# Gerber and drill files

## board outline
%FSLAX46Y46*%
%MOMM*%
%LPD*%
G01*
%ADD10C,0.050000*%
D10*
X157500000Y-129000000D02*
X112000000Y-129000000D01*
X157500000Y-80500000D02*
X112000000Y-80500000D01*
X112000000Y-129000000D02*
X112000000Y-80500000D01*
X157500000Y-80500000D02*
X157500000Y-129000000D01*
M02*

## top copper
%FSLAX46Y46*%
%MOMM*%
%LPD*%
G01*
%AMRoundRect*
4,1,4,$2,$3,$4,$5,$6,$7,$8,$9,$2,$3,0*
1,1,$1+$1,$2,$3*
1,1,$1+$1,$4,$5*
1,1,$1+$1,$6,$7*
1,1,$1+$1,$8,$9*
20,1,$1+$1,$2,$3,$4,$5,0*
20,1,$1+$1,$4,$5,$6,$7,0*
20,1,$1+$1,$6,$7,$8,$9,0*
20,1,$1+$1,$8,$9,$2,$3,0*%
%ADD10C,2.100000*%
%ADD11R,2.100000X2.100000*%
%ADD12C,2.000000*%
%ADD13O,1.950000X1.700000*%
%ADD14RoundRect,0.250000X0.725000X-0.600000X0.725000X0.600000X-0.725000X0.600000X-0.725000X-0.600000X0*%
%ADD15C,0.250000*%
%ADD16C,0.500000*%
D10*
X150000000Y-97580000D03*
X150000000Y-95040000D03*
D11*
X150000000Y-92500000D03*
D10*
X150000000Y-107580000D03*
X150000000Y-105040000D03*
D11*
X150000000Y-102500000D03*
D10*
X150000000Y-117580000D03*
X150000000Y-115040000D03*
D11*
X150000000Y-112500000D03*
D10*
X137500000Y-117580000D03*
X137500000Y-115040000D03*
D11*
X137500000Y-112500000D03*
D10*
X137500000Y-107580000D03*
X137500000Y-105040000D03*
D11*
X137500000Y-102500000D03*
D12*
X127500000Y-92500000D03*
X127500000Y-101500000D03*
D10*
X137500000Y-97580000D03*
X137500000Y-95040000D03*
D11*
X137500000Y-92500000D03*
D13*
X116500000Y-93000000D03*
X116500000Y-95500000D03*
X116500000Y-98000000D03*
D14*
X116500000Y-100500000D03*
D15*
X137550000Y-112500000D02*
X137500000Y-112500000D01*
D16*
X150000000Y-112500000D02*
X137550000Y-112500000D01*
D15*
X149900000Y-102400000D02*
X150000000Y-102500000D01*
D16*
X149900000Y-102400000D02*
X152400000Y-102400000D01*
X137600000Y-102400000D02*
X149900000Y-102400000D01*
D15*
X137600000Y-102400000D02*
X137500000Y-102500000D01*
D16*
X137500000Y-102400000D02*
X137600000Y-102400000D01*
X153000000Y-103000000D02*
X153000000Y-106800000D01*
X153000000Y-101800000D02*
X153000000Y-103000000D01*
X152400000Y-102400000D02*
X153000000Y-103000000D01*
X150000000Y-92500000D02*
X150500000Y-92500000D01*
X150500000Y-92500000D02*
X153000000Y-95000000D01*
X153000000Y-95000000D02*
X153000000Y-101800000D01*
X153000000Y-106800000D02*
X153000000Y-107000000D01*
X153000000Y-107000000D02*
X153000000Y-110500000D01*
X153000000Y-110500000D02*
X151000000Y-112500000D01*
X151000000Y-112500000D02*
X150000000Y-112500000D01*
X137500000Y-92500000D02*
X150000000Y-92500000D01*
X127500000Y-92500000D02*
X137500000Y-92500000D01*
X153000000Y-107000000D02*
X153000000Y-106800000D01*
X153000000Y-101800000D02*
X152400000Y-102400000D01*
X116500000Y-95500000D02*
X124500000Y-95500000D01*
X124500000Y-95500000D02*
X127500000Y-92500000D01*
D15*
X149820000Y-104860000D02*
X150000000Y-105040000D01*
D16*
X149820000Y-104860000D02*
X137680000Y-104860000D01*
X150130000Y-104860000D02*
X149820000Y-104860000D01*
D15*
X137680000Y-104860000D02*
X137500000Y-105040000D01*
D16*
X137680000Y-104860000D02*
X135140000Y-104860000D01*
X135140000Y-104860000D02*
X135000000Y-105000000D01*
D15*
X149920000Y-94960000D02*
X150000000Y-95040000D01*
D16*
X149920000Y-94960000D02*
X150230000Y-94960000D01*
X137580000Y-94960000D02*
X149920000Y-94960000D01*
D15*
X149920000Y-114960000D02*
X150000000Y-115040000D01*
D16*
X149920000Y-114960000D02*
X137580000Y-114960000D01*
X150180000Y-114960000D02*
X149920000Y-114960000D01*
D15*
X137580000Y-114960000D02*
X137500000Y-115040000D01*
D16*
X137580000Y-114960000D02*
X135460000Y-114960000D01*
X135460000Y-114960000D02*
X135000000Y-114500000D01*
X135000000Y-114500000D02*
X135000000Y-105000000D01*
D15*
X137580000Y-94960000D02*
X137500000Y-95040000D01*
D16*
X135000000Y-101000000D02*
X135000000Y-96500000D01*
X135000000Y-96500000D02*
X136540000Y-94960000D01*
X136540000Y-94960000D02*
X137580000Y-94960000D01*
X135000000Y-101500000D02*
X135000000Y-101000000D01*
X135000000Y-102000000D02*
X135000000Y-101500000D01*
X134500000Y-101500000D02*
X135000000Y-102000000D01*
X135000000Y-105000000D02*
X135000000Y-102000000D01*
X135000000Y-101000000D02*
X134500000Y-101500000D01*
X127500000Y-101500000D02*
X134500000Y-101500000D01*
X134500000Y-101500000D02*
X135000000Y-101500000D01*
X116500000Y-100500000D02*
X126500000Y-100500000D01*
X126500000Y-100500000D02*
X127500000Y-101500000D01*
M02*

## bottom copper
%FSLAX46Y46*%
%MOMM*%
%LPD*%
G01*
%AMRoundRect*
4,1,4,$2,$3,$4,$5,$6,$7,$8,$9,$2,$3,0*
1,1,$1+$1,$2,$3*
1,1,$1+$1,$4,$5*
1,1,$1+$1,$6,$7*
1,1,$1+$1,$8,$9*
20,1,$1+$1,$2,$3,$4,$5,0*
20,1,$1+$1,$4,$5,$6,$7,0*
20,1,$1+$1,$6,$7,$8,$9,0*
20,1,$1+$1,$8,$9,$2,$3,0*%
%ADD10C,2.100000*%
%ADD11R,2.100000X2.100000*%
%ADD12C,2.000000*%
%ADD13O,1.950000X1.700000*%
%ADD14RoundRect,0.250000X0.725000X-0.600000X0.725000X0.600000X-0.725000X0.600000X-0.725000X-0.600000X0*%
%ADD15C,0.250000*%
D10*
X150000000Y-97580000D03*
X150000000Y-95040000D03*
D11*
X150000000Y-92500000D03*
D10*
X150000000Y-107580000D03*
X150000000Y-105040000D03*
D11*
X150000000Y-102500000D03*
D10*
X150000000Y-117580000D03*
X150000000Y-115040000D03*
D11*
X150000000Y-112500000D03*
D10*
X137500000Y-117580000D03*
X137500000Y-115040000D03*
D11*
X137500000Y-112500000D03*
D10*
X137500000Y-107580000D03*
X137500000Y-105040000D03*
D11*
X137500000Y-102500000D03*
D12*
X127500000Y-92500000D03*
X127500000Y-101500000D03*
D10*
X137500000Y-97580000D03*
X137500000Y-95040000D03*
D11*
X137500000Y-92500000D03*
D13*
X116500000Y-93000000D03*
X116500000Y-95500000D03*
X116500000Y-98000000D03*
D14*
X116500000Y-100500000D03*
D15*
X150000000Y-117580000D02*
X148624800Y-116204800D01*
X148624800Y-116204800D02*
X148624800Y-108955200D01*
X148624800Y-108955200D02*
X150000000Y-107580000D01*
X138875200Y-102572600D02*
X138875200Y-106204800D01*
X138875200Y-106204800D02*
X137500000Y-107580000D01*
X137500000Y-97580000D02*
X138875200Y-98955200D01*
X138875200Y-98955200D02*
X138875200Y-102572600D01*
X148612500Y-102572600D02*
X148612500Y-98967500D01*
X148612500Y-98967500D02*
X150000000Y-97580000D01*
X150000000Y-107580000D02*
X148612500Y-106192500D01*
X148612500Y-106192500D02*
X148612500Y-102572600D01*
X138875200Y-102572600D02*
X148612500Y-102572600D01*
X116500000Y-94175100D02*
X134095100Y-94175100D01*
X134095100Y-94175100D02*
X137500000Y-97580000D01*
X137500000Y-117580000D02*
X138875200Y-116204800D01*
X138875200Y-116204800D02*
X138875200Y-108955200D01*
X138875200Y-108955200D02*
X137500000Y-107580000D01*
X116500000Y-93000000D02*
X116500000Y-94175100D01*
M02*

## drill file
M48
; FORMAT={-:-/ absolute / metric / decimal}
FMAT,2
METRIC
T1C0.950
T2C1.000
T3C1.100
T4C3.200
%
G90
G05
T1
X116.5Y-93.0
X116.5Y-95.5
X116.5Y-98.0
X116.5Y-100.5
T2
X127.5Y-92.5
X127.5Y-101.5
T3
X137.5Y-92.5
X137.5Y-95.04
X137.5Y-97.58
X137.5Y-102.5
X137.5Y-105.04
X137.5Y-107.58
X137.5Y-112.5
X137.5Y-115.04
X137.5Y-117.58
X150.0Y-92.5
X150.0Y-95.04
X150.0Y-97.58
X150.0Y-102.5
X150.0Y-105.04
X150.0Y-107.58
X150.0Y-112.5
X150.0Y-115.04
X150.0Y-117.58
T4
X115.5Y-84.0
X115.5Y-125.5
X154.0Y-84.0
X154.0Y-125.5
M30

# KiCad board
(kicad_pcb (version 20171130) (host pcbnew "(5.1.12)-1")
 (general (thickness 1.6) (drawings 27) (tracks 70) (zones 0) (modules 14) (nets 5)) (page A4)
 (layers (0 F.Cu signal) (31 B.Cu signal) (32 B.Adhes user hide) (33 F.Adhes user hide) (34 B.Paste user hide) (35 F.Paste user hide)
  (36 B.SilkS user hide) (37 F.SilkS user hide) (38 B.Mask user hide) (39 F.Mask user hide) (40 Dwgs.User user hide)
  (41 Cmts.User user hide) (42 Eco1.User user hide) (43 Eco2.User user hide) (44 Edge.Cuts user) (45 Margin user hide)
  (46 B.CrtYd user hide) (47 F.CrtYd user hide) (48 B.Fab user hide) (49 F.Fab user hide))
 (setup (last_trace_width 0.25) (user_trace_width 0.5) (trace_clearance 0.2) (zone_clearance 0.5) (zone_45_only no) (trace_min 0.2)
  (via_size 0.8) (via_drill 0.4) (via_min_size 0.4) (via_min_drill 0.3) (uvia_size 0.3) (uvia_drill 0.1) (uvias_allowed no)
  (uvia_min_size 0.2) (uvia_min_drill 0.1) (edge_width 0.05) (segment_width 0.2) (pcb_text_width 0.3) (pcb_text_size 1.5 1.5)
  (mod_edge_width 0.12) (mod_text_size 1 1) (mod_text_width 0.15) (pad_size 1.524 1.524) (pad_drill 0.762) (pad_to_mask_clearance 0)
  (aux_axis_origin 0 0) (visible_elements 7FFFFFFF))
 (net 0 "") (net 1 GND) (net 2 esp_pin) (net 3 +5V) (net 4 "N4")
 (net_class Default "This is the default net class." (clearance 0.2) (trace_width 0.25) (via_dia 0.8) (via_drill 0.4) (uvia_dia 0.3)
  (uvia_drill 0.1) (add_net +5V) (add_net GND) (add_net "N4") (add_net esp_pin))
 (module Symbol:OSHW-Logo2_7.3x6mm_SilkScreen (layer F.Cu) (at 137.5 124.5)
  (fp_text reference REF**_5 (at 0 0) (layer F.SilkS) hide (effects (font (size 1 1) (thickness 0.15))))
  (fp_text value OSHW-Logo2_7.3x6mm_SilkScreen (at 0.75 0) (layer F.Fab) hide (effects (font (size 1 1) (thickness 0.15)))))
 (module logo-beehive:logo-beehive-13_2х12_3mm (layer F.Cu) (at 123 109.22)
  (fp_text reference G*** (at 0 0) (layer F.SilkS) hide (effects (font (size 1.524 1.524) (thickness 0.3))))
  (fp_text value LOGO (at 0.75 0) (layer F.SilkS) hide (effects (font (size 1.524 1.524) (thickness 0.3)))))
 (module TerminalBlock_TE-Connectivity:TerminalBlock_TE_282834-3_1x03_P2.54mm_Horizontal (layer F.Cu) (at 150 92.5 270)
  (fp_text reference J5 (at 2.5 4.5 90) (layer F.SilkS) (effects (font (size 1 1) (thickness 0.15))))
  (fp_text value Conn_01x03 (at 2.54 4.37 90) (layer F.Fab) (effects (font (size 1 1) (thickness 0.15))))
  (pad 3 thru_hole circle (at 5.08 0 270) (size 2.1 2.1) (drill 1.1) (layers *.Cu *.Mask) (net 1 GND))
  (pad 2 thru_hole circle (at 2.54 0 270) (size 2.1 2.1) (drill 1.1) (layers *.Cu *.Mask) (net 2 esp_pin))
  (pad 1 thru_hole rect (at 0 0 270) (size 2.1 2.1) (drill 1.1) (layers *.Cu *.Mask) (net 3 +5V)))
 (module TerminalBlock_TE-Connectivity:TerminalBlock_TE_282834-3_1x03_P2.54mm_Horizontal (layer F.Cu) (at 150 102.5 270)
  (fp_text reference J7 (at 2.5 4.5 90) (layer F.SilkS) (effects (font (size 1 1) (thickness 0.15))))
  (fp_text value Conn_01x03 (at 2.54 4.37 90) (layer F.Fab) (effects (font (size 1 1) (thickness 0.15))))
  (pad 3 thru_hole circle (at 5.08 0 270) (size 2.1 2.1) (drill 1.1) (layers *.Cu *.Mask) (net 1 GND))
  (pad 2 thru_hole circle (at 2.54 0 270) (size 2.1 2.1) (drill 1.1) (layers *.Cu *.Mask) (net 2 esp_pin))
  (pad 1 thru_hole rect (at 0 0 270) (size 2.1 2.1) (drill 1.1) (layers *.Cu *.Mask) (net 3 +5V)))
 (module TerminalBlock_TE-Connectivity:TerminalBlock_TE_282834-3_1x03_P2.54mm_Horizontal (layer F.Cu) (at 150 112.5 270)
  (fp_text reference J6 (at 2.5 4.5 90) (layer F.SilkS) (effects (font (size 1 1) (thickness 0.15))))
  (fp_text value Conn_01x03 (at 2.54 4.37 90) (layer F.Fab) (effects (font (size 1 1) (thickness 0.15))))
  (pad 3 thru_hole circle (at 5.08 0 270) (size 2.1 2.1) (drill 1.1) (layers *.Cu *.Mask) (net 1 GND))
  (pad 2 thru_hole circle (at 2.54 0 270) (size 2.1 2.1) (drill 1.1) (layers *.Cu *.Mask) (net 2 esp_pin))
  (pad 1 thru_hole rect (at 0 0 270) (size 2.1 2.1) (drill 1.1) (layers *.Cu *.Mask) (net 3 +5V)))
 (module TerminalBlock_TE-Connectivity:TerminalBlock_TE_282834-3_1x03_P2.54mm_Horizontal (layer F.Cu) (at 137.5 112.5 270)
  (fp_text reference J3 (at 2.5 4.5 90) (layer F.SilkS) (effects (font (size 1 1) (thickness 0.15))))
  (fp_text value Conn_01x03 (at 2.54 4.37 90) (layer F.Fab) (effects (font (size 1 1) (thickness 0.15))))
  (pad 3 thru_hole circle (at 5.08 0 270) (size 2.1 2.1) (drill 1.1) (layers *.Cu *.Mask) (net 1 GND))
  (pad 2 thru_hole circle (at 2.54 0 270) (size 2.1 2.1) (drill 1.1) (layers *.Cu *.Mask) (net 2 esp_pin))
  (pad 1 thru_hole rect (at 0 0 270) (size 2.1 2.1) (drill 1.1) (layers *.Cu *.Mask) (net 3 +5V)))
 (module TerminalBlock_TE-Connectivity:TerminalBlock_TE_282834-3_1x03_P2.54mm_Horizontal (layer F.Cu) (at 137.5 102.5 270)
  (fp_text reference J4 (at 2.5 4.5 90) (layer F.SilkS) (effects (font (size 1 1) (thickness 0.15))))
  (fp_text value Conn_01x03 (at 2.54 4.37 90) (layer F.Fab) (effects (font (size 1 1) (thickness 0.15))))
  (pad 3 thru_hole circle (at 5.08 0 270) (size 2.1 2.1) (drill 1.1) (layers *.Cu *.Mask) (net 1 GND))
  (pad 2 thru_hole circle (at 2.54 0 270) (size 2.1 2.1) (drill 1.1) (layers *.Cu *.Mask) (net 2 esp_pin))
  (pad 1 thru_hole rect (at 0 0 270) (size 2.1 2.1) (drill 1.1) (layers *.Cu *.Mask) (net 3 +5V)))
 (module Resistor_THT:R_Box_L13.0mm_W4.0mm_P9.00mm (layer F.Cu) (at 127.5 101.5 90)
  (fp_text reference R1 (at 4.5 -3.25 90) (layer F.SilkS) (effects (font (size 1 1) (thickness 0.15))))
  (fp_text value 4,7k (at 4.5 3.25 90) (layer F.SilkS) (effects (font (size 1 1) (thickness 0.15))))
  (pad 2 thru_hole circle (at 9 0 90) (size 2 2) (drill 1) (layers *.Cu *.Mask) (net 3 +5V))
  (pad 1 thru_hole circle (at 0 0 90) (size 2 2) (drill 1) (layers *.Cu *.Mask) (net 2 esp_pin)))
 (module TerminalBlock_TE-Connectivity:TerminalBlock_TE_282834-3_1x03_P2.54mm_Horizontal (layer F.Cu) (at 137.5 92.5 270)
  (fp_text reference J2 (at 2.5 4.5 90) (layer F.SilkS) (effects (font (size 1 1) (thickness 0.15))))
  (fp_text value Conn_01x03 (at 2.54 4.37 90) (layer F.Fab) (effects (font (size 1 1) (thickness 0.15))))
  (pad 3 thru_hole circle (at 5.08 0 270) (size 2.1 2.1) (drill 1.1) (layers *.Cu *.Mask) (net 1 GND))
  (pad 2 thru_hole circle (at 2.54 0 270) (size 2.1 2.1) (drill 1.1) (layers *.Cu *.Mask) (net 2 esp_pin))
  (pad 1 thru_hole rect (at 0 0 270) (size 2.1 2.1) (drill 1.1) (layers *.Cu *.Mask) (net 3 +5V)))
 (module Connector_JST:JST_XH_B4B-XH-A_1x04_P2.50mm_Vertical (layer F.Cu) (at 116.5 100.5 90)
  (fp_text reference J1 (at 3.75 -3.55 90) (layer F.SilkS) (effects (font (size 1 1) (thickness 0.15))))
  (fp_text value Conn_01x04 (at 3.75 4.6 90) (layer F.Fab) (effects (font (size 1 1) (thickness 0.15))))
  (pad 4 thru_hole oval (at 7.5 0 90) (size 1.7 1.95) (drill 0.95) (layers *.Cu *.Mask) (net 1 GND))
  (pad 3 thru_hole oval (at 5 0 90) (size 1.7 1.95) (drill 0.95) (layers *.Cu *.Mask) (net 3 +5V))
  (pad 2 thru_hole oval (at 2.5 0 90) (size 1.7 1.95) (drill 0.95) (layers *.Cu *.Mask) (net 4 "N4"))
  (pad 1 thru_hole roundrect (at 0 0 90) (size 1.7 1.95) (drill 0.95) (layers *.Cu *.Mask) (roundrect_rratio 0.1470588235294118)
   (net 2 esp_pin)))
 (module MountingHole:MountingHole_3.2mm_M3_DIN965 (layer F.Cu) (at 154 125.5)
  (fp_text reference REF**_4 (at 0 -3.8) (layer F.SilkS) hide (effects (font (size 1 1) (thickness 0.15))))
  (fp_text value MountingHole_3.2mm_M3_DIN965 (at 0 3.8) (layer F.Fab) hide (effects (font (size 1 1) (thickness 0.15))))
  (pad 1 np_thru_hole circle (at 0 0) (size 3.2 3.2) (drill 3.2) (layers *.Cu *.Mask)))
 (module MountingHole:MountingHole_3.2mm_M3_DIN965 (layer F.Cu) (at 154 84)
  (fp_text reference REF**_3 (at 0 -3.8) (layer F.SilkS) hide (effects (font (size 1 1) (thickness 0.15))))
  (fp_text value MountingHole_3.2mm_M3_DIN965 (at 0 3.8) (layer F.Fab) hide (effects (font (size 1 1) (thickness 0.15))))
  (pad 1 np_thru_hole circle (at 0 0) (size 3.2 3.2) (drill 3.2) (layers *.Cu *.Mask)))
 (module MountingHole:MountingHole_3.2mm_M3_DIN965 (layer F.Cu) (at 115.5 125.5)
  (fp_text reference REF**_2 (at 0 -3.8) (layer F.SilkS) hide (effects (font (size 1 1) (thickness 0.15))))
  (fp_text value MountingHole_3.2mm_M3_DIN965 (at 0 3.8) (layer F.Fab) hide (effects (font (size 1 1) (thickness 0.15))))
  (pad 1 np_thru_hole circle (at 0 0) (size 3.2 3.2) (drill 3.2) (layers *.Cu *.Mask)))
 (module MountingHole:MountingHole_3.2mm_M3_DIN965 (layer F.Cu) (at 115.5 84)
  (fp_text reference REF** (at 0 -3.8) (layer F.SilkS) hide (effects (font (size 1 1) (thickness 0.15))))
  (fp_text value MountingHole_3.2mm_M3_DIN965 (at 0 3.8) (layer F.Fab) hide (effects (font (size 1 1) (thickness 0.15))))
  (pad 1 np_thru_hole circle (at 0 0) (size 3.2 3.2) (drill 3.2) (layers *.Cu *.Mask)))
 (gr_line (start 157.5 129) (end 112 129) (layer Edge.Cuts) (width 0.05))
 (gr_line (start 157.5 80.5) (end 112 80.5) (layer Edge.Cuts) (width 0.05))
 (gr_line (start 112 129) (end 112 80.5) (layer Edge.Cuts) (width 0.05))
 (gr_line (start 157.5 80.5) (end 157.5 129) (layer Edge.Cuts) (width 0.05))
 (segment (start 150 117.58) (end 148.6248 116.2048) (width 0.25) (layer B.Cu) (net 1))
 (segment (start 148.6248 116.2048) (end 148.6248 108.9552) (width 0.25) (layer B.Cu) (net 1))
 (segment (start 148.6248 108.9552) (end 150 107.58) (width 0.25) (layer B.Cu) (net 1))
 (segment (start 138.8752 102.5726) (end 138.8752 106.2048) (width 0.25) (layer B.Cu) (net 1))
 (segment (start 138.8752 106.2048) (end 137.5 107.58) (width 0.25) (layer B.Cu) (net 1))
 (segment (start 137.5 97.58) (end 138.8752 98.9552) (width 0.25) (layer B.Cu) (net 1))
 (segment (start 138.8752 98.9552) (end 138.8752 102.5726) (width 0.25) (layer B.Cu) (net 1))
 (segment (start 148.6125 102.5726) (end 148.6125 98.9675) (width 0.25) (layer B.Cu) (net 1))
 (segment (start 148.6125 98.9675) (end 150 97.58) (width 0.25) (layer B.Cu) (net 1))
 (segment (start 150 107.58) (end 148.6125 106.1925) (width 0.25) (layer B.Cu) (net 1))
 (segment (start 148.6125 106.1925) (end 148.6125 102.5726) (width 0.25) (layer B.Cu) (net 1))
 (segment (start 138.8752 102.5726) (end 148.6125 102.5726) (width 0.25) (layer B.Cu) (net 1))
 (segment (start 116.5 94.1751) (end 134.0951 94.1751) (width 0.25) (layer B.Cu) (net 1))
 (segment (start 134.0951 94.1751) (end 137.5 97.58) (width 0.25) (layer B.Cu) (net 1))
 (segment (start 137.5 117.58) (end 138.8752 116.2048) (width 0.25) (layer B.Cu) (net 1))
 (segment (start 138.8752 116.2048) (end 138.8752 108.9552) (width 0.25) (layer B.Cu) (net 1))
 (segment (start 138.8752 108.9552) (end 137.5 107.58) (width 0.25) (layer B.Cu) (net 1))
 (segment (start 116.5 93) (end 116.5 94.1751) (width 0.25) (layer B.Cu) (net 1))
 (segment (start 137.55 112.5) (end 137.5 112.5) (width 0.25) (layer F.Cu) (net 3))
 (segment (start 150 112.5) (end 137.55 112.5) (width 0.5) (layer F.Cu) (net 3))
 (segment (start 149.9 102.4) (end 150 102.5) (width 0.25) (layer F.Cu) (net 3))
 (segment (start 149.9 102.4) (end 152.4 102.4) (width 0.5) (layer F.Cu) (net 3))
 (segment (start 137.6 102.4) (end 149.9 102.4) (width 0.5) (layer F.Cu) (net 3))
 (segment (start 137.6 102.4) (end 137.5 102.5) (width 0.25) (layer F.Cu) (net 3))
 (segment (start 137.5 102.4) (end 137.6 102.4) (width 0.5) (layer F.Cu) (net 3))
 (segment (start 153 103) (end 153 106.8) (width 0.5) (layer F.Cu) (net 3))
 (segment (start 153 101.8) (end 153 103) (width 0.5) (layer F.Cu) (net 3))
 (segment (start 152.4 102.4) (end 153 103) (width 0.5) (layer F.Cu) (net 3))
 (segment (start 150 92.5) (end 150.5 92.5) (width 0.5) (layer F.Cu) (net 3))
 (segment (start 150.5 92.5) (end 153 95) (width 0.5) (layer F.Cu) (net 3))
 (segment (start 153 95) (end 153 101.8) (width 0.5) (layer F.Cu) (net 3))
 (segment (start 153 106.8) (end 153 107) (width 0.5) (layer F.Cu) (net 3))
 (segment (start 153 107) (end 153 110.5) (width 0.5) (layer F.Cu) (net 3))
 (segment (start 153 110.5) (end 151 112.5) (width 0.5) (layer F.Cu) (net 3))
 (segment (start 151 112.5) (end 150 112.5) (width 0.5) (layer F.Cu) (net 3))
 (segment (start 137.5 92.5) (end 150 92.5) (width 0.5) (layer F.Cu) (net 3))
 (segment (start 127.5 92.5) (end 137.5 92.5) (width 0.5) (layer F.Cu) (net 3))
 (segment (start 153 107) (end 153 106.8) (width 0.5) (layer F.Cu) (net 3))
 (segment (start 153 101.8) (end 152.4 102.4) (width 0.5) (layer F.Cu) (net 3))
 (segment (start 116.5 95.5) (end 124.5 95.5) (width 0.5) (layer F.Cu) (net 3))
 (segment (start 124.5 95.5) (end 127.5 92.5) (width 0.5) (layer F.Cu) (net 3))
 (segment (start 149.82 104.86) (end 150 105.04) (width 0.25) (layer F.Cu) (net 2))
 (segment (start 149.82 104.86) (end 137.68 104.86) (width 0.5) (layer F.Cu) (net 2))
 (segment (start 150.13 104.86) (end 149.82 104.86) (width 0.5) (layer F.Cu) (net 2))
 (segment (start 137.68 104.86) (end 137.5 105.04) (width 0.25) (layer F.Cu) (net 2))
 (segment (start 137.68 104.86) (end 135.14 104.86) (width 0.5) (layer F.Cu) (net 2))
 (segment (start 135.14 104.86) (end 135 105) (width 0.5) (layer F.Cu) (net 2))
 (segment (start 149.92 94.96) (end 150 95.04) (width 0.25) (layer F.Cu) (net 2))
 (segment (start 149.92 94.96) (end 150.23 94.96) (width 0.5) (layer F.Cu) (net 2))
 (segment (start 137.58 94.96) (end 149.92 94.96) (width 0.5) (layer F.Cu) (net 2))
 (segment (start 149.92 114.96) (end 150 115.04) (width 0.25) (layer F.Cu) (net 2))
 (segment (start 149.92 114.96) (end 137.58 114.96) (width 0.5) (layer F.Cu) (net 2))
 (segment (start 150.18 114.96) (end 149.92 114.96) (width 0.5) (layer F.Cu) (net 2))
 (segment (start 137.58 114.96) (end 137.5 115.04) (width 0.25) (layer F.Cu) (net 2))
 (segment (start 137.58 114.96) (end 135.46 114.96) (width 0.5) (layer F.Cu) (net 2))
 (segment (start 135.46 114.96) (end 135 114.5) (width 0.5) (layer F.Cu) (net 2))
 (segment (start 135 114.5) (end 135 105) (width 0.5) (layer F.Cu) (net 2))
 (segment (start 137.58 94.96) (end 137.5 95.04) (width 0.25) (layer F.Cu) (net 2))
 (segment (start 135 101) (end 135 96.5) (width 0.5) (layer F.Cu) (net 2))
 (segment (start 135 96.5) (end 136.54 94.96) (width 0.5) (layer F.Cu) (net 2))
 (segment (start 136.54 94.96) (end 137.58 94.96) (width 0.5) (layer F.Cu) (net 2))
 (segment (start 135 101.5) (end 135 101) (width 0.5) (layer F.Cu) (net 2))
 (segment (start 135 102) (end 135 101.5) (width 0.5) (layer F.Cu) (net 2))
 (segment (start 134.5 101.5) (end 135 102) (width 0.5) (layer F.Cu) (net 2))
 (segment (start 135 105) (end 135 102) (width 0.5) (layer F.Cu) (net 2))
 (segment (start 135 101) (end 134.5 101.5) (width 0.5) (layer F.Cu) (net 2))
 (segment (start 127.5 101.5) (end 134.5 101.5) (width 0.5) (layer F.Cu) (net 2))
 (segment (start 134.5 101.5) (end 135 101.5) (width 0.5) (layer F.Cu) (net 2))
 (segment (start 116.5 100.5) (end 126.5 100.5) (width 0.5) (layer F.Cu) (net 2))
 (segment (start 126.5 100.5) (end 127.5 101.5) (width 0.5) (layer F.Cu) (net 2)))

